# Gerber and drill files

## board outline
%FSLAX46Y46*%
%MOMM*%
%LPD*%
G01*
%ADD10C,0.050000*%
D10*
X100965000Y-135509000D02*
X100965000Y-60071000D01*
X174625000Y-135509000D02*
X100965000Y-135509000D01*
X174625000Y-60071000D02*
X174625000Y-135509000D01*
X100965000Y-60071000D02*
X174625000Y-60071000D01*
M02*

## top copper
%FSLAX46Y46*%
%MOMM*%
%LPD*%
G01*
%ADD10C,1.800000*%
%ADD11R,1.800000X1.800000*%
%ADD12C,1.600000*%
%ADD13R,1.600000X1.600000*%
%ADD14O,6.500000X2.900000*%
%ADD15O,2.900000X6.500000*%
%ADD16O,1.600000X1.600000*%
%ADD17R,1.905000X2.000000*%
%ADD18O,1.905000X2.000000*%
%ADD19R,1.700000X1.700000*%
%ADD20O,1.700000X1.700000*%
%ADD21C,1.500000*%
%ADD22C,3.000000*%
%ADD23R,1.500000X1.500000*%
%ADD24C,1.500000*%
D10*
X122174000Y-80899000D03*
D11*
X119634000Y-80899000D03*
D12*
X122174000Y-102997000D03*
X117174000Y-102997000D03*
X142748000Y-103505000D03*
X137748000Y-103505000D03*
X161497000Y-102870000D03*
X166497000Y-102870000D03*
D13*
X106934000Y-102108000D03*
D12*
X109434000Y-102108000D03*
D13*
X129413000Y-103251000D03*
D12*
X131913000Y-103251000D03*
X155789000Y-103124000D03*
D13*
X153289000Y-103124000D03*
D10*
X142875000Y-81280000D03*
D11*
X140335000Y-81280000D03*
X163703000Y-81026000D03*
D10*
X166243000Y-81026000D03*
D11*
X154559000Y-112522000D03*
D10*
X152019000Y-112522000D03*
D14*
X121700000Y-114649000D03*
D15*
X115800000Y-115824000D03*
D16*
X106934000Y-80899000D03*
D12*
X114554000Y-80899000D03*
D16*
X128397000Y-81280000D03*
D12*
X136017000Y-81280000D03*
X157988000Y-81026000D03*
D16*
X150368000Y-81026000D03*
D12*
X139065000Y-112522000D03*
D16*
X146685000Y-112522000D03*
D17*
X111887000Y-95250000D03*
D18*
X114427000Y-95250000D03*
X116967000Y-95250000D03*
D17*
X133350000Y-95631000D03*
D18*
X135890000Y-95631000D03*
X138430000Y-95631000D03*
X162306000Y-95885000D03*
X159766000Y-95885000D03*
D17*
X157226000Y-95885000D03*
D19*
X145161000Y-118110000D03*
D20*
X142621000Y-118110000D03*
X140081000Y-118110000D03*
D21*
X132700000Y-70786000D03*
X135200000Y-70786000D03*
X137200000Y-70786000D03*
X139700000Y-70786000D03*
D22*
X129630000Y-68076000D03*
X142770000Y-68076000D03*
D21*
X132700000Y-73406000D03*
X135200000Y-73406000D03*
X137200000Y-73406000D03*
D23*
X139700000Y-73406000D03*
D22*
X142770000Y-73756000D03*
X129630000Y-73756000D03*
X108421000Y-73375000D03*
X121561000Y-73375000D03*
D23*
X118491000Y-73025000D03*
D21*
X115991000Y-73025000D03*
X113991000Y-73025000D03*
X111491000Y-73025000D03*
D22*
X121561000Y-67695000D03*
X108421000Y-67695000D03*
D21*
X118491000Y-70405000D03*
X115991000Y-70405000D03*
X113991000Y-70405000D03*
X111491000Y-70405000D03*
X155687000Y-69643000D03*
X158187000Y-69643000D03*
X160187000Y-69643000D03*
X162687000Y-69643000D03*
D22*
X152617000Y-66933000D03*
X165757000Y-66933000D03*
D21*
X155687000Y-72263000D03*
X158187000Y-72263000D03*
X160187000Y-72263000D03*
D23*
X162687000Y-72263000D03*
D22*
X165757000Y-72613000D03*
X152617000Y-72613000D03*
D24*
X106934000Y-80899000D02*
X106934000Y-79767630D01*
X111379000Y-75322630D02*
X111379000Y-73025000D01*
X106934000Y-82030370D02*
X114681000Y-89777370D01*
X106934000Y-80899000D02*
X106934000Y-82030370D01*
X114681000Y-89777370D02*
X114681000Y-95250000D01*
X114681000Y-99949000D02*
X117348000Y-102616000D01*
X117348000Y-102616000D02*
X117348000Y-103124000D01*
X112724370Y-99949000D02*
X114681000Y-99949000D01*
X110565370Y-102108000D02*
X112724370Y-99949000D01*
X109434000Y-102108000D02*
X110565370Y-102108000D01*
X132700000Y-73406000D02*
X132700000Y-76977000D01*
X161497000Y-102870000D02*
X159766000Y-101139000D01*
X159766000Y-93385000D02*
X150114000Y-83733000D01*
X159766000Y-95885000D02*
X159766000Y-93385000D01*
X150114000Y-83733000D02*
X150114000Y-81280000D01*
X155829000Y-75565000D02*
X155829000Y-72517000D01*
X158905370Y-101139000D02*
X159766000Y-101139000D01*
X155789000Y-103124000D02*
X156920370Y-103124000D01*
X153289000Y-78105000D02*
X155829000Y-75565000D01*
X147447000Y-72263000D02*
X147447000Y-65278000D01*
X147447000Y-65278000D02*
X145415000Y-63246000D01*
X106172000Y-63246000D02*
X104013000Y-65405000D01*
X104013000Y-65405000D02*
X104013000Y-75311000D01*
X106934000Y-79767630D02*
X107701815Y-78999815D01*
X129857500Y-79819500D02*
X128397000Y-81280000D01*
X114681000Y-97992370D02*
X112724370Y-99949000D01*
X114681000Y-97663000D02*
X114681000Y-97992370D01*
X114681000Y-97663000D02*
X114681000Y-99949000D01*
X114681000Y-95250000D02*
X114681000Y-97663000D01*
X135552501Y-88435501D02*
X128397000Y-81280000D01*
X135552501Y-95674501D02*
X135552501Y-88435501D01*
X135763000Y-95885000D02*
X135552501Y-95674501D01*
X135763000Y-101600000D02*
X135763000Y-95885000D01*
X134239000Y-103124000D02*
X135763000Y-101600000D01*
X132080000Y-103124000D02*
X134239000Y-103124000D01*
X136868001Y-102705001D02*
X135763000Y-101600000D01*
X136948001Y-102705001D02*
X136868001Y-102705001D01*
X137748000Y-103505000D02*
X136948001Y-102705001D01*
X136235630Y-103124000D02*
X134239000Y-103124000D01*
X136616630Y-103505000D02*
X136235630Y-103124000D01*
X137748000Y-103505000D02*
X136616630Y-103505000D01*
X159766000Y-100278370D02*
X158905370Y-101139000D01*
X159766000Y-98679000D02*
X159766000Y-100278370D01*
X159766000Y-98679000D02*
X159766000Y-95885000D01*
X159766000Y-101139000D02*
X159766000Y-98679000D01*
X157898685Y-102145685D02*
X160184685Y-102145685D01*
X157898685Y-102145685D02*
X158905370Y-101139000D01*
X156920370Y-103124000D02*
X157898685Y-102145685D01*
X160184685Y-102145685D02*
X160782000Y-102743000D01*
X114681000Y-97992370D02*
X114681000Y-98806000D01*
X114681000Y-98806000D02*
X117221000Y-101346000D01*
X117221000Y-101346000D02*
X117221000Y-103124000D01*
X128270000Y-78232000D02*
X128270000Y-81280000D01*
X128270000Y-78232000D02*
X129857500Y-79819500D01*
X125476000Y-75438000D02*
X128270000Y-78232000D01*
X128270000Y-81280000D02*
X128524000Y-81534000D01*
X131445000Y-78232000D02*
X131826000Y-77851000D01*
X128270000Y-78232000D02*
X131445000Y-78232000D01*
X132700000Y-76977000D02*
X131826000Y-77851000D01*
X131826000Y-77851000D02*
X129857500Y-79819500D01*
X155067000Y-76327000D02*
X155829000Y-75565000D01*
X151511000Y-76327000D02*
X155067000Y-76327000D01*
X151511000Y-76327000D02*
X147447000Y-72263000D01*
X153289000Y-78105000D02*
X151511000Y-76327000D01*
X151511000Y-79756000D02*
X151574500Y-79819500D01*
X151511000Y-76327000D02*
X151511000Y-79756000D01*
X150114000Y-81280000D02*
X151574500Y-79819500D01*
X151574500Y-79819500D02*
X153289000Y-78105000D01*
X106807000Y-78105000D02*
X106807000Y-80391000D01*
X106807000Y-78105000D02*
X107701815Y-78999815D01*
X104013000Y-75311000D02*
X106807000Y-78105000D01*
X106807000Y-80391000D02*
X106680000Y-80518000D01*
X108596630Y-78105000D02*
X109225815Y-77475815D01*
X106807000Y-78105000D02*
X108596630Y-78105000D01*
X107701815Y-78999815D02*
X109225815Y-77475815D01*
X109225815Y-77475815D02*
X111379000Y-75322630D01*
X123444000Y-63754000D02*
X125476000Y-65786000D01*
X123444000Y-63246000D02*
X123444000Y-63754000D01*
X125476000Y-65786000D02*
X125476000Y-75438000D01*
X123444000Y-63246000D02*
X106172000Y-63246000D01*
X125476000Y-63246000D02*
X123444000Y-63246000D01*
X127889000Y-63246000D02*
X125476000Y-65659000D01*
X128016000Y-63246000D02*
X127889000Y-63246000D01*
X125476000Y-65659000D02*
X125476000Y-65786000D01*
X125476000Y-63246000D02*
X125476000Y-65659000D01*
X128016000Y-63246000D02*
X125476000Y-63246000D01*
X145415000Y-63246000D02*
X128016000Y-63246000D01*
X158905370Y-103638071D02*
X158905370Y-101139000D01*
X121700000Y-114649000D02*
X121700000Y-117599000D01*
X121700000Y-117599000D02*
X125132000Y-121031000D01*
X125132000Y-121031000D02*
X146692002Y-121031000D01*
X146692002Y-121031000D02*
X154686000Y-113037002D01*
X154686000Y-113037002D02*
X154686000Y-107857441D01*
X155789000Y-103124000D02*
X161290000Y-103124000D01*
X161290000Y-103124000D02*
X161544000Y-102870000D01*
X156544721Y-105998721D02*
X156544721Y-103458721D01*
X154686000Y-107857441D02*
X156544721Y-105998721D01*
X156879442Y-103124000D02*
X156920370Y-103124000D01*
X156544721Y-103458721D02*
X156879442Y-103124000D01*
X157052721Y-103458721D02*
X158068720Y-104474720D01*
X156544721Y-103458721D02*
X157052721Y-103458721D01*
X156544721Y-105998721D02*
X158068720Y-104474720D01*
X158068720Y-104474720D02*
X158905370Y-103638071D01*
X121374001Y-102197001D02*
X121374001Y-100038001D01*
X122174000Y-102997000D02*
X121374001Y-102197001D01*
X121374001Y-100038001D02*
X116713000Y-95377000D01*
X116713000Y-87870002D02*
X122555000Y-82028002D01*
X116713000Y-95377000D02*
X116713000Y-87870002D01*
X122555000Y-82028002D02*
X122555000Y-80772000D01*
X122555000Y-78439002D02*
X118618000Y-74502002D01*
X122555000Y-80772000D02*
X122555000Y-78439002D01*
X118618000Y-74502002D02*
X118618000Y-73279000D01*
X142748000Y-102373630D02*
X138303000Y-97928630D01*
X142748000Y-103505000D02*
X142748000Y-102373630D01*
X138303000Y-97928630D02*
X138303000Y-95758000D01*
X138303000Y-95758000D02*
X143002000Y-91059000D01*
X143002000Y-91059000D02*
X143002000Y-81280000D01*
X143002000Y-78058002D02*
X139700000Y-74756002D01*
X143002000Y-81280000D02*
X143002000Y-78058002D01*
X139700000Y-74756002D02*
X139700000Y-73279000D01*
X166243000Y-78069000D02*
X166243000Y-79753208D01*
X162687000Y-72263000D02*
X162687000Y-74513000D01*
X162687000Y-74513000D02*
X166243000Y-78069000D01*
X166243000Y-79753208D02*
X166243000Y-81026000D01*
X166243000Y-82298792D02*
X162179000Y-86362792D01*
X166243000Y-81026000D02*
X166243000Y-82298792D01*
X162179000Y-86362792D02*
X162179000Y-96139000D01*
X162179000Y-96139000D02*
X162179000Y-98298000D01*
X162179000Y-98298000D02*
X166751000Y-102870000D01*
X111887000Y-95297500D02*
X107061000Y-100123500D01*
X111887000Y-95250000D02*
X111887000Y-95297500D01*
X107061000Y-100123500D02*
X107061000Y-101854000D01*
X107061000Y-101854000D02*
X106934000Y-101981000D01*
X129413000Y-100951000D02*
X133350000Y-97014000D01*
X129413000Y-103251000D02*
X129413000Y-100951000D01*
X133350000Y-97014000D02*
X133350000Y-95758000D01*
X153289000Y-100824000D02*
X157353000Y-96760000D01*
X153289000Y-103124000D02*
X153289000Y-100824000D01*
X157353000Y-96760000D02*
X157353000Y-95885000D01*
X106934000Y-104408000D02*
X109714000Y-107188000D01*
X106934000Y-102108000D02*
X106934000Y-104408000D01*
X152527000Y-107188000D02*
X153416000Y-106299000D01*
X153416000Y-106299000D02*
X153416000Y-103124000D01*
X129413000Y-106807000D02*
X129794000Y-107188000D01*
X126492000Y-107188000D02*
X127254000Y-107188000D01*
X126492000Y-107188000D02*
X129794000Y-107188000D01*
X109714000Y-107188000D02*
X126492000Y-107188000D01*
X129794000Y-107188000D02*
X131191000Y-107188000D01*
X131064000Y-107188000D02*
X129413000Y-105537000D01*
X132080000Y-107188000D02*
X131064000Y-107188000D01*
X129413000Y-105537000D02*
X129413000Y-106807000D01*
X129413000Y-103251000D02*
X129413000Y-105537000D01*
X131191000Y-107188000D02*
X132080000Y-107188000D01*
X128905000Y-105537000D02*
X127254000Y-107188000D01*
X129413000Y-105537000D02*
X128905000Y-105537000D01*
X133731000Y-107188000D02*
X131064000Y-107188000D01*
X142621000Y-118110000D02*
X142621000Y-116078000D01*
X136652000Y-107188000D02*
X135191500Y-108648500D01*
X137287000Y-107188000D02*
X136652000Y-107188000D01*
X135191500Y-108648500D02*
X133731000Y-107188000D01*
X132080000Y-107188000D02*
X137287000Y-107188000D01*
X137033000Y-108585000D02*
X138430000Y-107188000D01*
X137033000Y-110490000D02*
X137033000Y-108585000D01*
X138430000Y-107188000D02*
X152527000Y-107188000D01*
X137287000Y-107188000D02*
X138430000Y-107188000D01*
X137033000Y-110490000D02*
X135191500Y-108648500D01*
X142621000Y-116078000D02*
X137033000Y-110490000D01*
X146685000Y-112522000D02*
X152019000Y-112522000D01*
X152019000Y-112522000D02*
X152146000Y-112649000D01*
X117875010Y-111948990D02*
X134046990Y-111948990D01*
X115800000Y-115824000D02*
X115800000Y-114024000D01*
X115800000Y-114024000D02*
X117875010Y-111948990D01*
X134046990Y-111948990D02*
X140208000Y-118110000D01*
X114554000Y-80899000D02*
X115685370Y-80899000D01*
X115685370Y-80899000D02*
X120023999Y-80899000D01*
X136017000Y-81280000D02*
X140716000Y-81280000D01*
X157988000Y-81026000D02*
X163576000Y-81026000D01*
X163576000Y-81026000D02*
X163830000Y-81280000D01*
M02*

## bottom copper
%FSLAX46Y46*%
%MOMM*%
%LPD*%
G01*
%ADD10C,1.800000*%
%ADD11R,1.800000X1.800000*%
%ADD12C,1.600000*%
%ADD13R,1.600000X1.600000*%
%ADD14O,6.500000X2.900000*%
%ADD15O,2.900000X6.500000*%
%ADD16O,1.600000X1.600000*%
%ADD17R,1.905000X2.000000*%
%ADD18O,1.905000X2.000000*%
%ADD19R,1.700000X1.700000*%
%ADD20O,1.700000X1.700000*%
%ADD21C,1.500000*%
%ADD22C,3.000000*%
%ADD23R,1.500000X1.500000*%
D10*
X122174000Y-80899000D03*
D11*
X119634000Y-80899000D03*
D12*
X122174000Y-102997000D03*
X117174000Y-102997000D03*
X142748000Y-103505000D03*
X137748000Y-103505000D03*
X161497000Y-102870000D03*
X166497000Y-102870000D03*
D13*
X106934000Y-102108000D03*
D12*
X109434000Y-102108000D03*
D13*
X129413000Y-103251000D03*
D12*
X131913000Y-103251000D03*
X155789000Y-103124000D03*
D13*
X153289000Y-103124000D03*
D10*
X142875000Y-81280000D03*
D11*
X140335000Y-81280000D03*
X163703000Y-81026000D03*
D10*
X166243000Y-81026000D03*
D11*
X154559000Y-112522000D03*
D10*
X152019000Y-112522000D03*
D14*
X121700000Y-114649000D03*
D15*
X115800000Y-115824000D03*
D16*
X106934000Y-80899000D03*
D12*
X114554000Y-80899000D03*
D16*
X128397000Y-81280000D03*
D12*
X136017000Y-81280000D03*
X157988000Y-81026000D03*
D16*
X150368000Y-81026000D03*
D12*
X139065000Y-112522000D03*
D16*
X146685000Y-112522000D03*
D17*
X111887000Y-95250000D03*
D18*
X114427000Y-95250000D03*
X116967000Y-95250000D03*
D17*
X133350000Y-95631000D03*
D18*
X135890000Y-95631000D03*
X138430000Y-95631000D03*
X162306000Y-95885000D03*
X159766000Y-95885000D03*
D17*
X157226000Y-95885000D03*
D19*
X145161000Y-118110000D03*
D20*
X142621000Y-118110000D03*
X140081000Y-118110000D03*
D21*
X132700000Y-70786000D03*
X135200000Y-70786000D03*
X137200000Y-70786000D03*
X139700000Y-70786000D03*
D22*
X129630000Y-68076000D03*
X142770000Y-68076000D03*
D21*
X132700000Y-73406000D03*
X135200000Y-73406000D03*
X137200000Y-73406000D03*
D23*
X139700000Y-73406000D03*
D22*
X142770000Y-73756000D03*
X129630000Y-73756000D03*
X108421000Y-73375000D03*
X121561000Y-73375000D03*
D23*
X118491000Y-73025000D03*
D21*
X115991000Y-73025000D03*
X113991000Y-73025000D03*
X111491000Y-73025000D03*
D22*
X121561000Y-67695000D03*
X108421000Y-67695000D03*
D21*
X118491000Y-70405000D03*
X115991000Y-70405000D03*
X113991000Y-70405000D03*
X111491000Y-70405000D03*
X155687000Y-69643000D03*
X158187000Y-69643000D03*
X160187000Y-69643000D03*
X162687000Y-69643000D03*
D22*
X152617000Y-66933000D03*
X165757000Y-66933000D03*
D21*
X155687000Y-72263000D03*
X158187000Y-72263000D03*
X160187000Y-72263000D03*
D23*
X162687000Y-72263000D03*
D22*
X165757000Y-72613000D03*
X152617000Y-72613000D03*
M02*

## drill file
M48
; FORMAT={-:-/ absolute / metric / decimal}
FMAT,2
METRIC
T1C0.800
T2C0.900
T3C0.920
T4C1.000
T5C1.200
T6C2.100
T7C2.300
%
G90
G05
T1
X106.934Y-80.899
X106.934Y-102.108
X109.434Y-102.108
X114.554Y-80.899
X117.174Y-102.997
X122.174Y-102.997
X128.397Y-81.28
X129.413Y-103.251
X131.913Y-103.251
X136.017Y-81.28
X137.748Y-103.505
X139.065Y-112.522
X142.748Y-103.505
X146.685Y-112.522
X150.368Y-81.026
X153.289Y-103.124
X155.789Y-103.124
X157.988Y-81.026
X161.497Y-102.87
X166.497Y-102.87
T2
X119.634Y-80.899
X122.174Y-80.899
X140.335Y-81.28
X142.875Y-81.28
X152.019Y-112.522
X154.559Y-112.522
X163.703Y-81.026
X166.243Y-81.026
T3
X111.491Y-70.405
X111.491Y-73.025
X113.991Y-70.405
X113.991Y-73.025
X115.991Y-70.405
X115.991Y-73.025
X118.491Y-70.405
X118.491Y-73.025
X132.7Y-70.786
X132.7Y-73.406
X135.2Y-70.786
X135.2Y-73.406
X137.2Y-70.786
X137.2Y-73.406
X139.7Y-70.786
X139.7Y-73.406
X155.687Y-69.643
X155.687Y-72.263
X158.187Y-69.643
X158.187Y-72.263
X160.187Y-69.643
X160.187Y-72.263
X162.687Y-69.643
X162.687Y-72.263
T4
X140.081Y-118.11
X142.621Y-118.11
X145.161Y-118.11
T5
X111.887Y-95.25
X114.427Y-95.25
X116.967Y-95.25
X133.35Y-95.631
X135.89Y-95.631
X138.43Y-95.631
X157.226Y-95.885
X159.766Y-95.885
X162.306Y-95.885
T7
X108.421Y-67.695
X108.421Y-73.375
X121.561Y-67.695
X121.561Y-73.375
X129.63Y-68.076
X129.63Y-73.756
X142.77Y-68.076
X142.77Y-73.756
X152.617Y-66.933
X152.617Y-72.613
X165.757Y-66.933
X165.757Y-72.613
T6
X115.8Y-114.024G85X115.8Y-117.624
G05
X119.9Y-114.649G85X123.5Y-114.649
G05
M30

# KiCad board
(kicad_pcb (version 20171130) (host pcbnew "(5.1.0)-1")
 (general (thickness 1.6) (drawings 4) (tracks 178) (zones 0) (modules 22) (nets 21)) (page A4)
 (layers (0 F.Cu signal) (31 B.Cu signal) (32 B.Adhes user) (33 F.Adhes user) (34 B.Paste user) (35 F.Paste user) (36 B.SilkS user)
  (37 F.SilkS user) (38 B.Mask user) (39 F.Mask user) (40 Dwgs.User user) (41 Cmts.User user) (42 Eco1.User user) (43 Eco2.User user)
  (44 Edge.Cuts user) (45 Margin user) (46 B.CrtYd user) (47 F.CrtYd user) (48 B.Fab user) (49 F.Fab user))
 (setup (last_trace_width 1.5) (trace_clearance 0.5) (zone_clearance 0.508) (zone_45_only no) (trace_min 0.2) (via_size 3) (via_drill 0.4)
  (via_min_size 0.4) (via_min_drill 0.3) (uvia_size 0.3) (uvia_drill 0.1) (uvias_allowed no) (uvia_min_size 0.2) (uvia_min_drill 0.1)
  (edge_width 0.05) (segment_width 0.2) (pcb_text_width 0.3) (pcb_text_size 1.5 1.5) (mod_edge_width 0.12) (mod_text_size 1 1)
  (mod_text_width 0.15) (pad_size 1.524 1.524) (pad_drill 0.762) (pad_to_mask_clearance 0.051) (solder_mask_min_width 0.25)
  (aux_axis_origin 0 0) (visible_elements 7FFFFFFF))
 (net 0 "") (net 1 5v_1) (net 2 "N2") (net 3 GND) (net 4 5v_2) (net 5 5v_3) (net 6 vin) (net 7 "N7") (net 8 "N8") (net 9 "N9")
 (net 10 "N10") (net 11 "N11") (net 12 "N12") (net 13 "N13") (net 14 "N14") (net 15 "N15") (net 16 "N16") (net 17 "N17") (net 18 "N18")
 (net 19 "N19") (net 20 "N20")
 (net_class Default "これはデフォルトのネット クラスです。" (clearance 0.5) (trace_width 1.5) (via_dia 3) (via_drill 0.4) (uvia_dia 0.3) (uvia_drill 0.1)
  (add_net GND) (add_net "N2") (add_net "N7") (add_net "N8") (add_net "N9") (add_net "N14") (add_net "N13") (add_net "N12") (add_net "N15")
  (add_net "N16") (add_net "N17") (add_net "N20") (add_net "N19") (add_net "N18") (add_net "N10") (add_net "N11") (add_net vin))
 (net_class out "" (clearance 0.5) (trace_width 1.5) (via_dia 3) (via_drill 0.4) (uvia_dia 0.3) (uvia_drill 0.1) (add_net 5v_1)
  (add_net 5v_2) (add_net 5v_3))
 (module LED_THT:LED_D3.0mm (layer F.Cu) (at 119.634 80.899)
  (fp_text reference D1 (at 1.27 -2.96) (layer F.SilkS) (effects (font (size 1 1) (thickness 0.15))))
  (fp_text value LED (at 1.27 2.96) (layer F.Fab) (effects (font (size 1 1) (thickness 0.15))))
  (pad 2 thru_hole circle (at 2.54 0) (size 1.8 1.8) (drill 0.9) (layers *.Cu *.Mask) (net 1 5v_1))
  (pad 1 thru_hole rect (at 0 0) (size 1.8 1.8) (drill 0.9) (layers *.Cu *.Mask) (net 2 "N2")))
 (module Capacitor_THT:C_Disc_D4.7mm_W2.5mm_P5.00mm (layer F.Cu) (at 122.174 102.997 180)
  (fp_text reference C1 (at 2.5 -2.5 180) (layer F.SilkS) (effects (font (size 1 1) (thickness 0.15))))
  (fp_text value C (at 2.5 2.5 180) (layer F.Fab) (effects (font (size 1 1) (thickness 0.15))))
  (pad 1 thru_hole circle (at 0 0 180) (size 1.6 1.6) (drill 0.8) (layers *.Cu *.Mask) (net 1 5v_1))
  (pad 2 thru_hole circle (at 5 0 180) (size 1.6 1.6) (drill 0.8) (layers *.Cu *.Mask) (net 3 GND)))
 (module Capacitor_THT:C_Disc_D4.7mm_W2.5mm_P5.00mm (layer F.Cu) (at 142.748 103.505 180)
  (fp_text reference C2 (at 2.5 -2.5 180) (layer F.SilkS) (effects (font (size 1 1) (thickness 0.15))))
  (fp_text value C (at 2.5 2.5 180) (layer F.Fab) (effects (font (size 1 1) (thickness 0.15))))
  (pad 1 thru_hole circle (at 0 0 180) (size 1.6 1.6) (drill 0.8) (layers *.Cu *.Mask) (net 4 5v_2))
  (pad 2 thru_hole circle (at 5 0 180) (size 1.6 1.6) (drill 0.8) (layers *.Cu *.Mask) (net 3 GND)))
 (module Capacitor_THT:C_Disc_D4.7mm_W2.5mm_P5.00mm (layer F.Cu) (at 166.497 102.87 180)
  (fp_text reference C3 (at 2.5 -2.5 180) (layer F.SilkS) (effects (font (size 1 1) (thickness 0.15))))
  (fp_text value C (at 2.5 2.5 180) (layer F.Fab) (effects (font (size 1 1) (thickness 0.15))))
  (pad 2 thru_hole circle (at 5 0 180) (size 1.6 1.6) (drill 0.8) (layers *.Cu *.Mask) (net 3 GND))
  (pad 1 thru_hole circle (at 0 0 180) (size 1.6 1.6) (drill 0.8) (layers *.Cu *.Mask) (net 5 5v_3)))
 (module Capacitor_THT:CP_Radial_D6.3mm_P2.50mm (layer F.Cu) (at 106.934 102.108)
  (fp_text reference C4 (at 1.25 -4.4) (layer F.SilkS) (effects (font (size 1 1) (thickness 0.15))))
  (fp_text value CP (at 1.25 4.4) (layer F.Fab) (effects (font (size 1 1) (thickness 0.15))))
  (pad 1 thru_hole rect (at 0 0) (size 1.6 1.6) (drill 0.8) (layers *.Cu *.Mask) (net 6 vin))
  (pad 2 thru_hole circle (at 2.5 0) (size 1.6 1.6) (drill 0.8) (layers *.Cu *.Mask) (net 3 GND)))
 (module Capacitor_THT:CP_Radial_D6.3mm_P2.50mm (layer F.Cu) (at 129.413 103.251)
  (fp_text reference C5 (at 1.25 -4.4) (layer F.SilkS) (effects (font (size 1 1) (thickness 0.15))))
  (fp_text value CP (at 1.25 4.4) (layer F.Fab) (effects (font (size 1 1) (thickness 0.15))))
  (pad 1 thru_hole rect (at 0 0) (size 1.6 1.6) (drill 0.8) (layers *.Cu *.Mask) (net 6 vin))
  (pad 2 thru_hole circle (at 2.5 0) (size 1.6 1.6) (drill 0.8) (layers *.Cu *.Mask) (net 3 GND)))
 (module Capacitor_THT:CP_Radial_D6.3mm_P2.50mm (layer F.Cu) (at 153.289 103.124)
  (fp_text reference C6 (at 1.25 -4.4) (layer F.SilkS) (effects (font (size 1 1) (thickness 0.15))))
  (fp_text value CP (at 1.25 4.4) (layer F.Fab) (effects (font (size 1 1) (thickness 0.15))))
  (pad 2 thru_hole circle (at 2.5 0) (size 1.6 1.6) (drill 0.8) (layers *.Cu *.Mask) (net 3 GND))
  (pad 1 thru_hole rect (at 0 0) (size 1.6 1.6) (drill 0.8) (layers *.Cu *.Mask) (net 6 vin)))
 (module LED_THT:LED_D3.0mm (layer F.Cu) (at 140.335 81.28)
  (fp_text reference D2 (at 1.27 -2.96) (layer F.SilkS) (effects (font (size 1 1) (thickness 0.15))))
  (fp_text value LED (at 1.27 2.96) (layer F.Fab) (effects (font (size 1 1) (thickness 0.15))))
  (pad 2 thru_hole circle (at 2.54 0) (size 1.8 1.8) (drill 0.9) (layers *.Cu *.Mask) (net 4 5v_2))
  (pad 1 thru_hole rect (at 0 0) (size 1.8 1.8) (drill 0.9) (layers *.Cu *.Mask) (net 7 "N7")))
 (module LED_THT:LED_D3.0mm (layer F.Cu) (at 163.703 81.026)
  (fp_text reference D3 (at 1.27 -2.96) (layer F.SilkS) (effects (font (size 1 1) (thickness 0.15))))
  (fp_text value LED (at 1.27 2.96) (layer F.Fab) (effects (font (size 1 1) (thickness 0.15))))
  (pad 1 thru_hole rect (at 0 0) (size 1.8 1.8) (drill 0.9) (layers *.Cu *.Mask) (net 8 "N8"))
  (pad 2 thru_hole circle (at 2.54 0) (size 1.8 1.8) (drill 0.9) (layers *.Cu *.Mask) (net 5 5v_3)))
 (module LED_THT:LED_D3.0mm (layer F.Cu) (at 154.559 112.522 180)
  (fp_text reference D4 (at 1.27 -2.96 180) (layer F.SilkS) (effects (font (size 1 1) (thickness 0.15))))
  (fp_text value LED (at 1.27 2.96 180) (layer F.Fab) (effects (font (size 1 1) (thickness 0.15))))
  (pad 1 thru_hole rect (at 0 0 180) (size 1.8 1.8) (drill 0.9) (layers *.Cu *.Mask) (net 3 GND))
  (pad 2 thru_hole circle (at 2.54 0 180) (size 1.8 1.8) (drill 0.9) (layers *.Cu *.Mask) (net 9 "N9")))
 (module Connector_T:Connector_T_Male (layer F.Cu) (at 114.3 115.824)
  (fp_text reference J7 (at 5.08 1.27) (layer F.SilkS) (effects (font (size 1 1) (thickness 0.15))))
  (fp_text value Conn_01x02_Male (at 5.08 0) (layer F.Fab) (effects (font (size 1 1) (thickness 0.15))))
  (pad 2 thru_hole oval (at 7.4 -1.175) (size 6.5 2.9) (drill oval 5.7 2.1) (layers *.Cu *.Mask) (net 3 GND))
  (pad 1 thru_hole oval (at 1.5 0) (size 2.9 6.5) (drill oval 2.1 5.7) (layers *.Cu *.Mask) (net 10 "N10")))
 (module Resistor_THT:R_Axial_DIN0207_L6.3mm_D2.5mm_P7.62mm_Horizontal (layer F.Cu) (at 114.554 80.899 180)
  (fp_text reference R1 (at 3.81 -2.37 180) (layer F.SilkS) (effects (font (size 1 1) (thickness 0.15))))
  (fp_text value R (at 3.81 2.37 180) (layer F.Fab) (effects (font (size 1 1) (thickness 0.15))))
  (pad 2 thru_hole oval (at 7.62 0 180) (size 1.6 1.6) (drill 0.8) (layers *.Cu *.Mask) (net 3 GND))
  (pad 1 thru_hole circle (at 0 0 180) (size 1.6 1.6) (drill 0.8) (layers *.Cu *.Mask) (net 2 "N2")))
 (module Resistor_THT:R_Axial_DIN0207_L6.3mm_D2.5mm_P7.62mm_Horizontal (layer F.Cu) (at 136.017 81.28 180)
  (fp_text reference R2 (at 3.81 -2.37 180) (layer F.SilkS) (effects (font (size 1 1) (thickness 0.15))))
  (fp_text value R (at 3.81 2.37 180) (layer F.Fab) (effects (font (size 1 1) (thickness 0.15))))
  (pad 2 thru_hole oval (at 7.62 0 180) (size 1.6 1.6) (drill 0.8) (layers *.Cu *.Mask) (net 3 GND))
  (pad 1 thru_hole circle (at 0 0 180) (size 1.6 1.6) (drill 0.8) (layers *.Cu *.Mask) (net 7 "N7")))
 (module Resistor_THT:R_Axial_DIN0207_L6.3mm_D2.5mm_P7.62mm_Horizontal (layer F.Cu) (at 157.988 81.026 180)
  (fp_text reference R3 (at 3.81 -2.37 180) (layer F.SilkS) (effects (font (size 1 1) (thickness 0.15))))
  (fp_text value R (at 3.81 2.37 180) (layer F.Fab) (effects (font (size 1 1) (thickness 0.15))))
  (pad 1 thru_hole circle (at 0 0 180) (size 1.6 1.6) (drill 0.8) (layers *.Cu *.Mask) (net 8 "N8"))
  (pad 2 thru_hole oval (at 7.62 0 180) (size 1.6 1.6) (drill 0.8) (layers *.Cu *.Mask) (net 3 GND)))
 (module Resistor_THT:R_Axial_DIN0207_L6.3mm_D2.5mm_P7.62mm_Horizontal (layer F.Cu) (at 139.065 112.522)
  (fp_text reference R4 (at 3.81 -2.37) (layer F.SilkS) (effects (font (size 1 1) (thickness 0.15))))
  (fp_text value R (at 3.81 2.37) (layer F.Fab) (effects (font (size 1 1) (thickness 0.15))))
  (pad 1 thru_hole circle (at 0 0) (size 1.6 1.6) (drill 0.8) (layers *.Cu *.Mask) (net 6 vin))
  (pad 2 thru_hole oval (at 7.62 0) (size 1.6 1.6) (drill 0.8) (layers *.Cu *.Mask) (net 9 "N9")))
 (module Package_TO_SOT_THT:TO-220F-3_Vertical (layer F.Cu) (at 111.887 95.25)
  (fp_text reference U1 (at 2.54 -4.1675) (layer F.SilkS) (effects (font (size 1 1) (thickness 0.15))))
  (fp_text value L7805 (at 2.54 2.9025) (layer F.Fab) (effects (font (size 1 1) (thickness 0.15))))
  (pad 1 thru_hole rect (at 0 0) (size 1.905 2) (drill 1.2) (layers *.Cu *.Mask) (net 6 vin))
  (pad 2 thru_hole oval (at 2.54 0) (size 1.905 2) (drill 1.2) (layers *.Cu *.Mask) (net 3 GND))
  (pad 3 thru_hole oval (at 5.08 0) (size 1.905 2) (drill 1.2) (layers *.Cu *.Mask) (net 1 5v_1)))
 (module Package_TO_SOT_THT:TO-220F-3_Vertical (layer F.Cu) (at 133.35 95.631)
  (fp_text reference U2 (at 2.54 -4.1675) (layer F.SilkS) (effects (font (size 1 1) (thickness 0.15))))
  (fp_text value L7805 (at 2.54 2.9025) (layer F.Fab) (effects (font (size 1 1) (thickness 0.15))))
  (pad 1 thru_hole rect (at 0 0) (size 1.905 2) (drill 1.2) (layers *.Cu *.Mask) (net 6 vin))
  (pad 2 thru_hole oval (at 2.54 0) (size 1.905 2) (drill 1.2) (layers *.Cu *.Mask) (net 3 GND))
  (pad 3 thru_hole oval (at 5.08 0) (size 1.905 2) (drill 1.2) (layers *.Cu *.Mask) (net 4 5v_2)))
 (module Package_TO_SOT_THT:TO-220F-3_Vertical (layer F.Cu) (at 157.226 95.885)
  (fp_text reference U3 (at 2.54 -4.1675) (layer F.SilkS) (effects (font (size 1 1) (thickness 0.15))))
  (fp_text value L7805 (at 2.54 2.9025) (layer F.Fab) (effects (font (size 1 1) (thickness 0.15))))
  (pad 3 thru_hole oval (at 5.08 0) (size 1.905 2) (drill 1.2) (layers *.Cu *.Mask) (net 5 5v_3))
  (pad 2 thru_hole oval (at 2.54 0) (size 1.905 2) (drill 1.2) (layers *.Cu *.Mask) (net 3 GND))
  (pad 1 thru_hole rect (at 0 0) (size 1.905 2) (drill 1.2) (layers *.Cu *.Mask) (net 6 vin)))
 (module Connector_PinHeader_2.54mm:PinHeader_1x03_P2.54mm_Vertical (layer F.Cu) (at 145.161 118.11 270)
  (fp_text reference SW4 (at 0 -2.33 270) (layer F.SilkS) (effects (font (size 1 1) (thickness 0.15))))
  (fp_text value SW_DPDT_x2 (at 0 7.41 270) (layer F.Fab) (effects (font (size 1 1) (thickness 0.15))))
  (pad 1 thru_hole rect (at 0 0 270) (size 1.7 1.7) (drill 1) (layers *.Cu *.Mask) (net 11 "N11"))
  (pad 2 thru_hole oval (at 0 2.54 270) (size 1.7 1.7) (drill 1) (layers *.Cu *.Mask) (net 6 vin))
  (pad 3 thru_hole oval (at 0 5.08 270) (size 1.7 1.7) (drill 1) (layers *.Cu *.Mask) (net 10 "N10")))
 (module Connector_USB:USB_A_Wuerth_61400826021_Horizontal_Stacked (layer F.Cu) (at 139.7 73.406 180)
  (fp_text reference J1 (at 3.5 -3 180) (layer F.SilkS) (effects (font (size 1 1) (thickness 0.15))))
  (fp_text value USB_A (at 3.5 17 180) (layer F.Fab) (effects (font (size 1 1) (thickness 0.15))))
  (pad 8 thru_hole circle (at 7 2.62 180) (size 1.5 1.5) (drill 0.92) (layers *.Cu *.Mask))
  (pad 7 thru_hole circle (at 4.5 2.62 180) (size 1.5 1.5) (drill 0.92) (layers *.Cu *.Mask))
  (pad 6 thru_hole circle (at 2.5 2.62 180) (size 1.5 1.5) (drill 0.92) (layers *.Cu *.Mask))
  (pad 5 thru_hole circle (at 0 2.62 180) (size 1.5 1.5) (drill 0.92) (layers *.Cu *.Mask) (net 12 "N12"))
  (pad 9 thru_hole circle (at 10.07 5.33 180) (size 3 3) (drill 2.3) (layers *.Cu *.Mask))
  (pad 9 thru_hole circle (at -3.07 5.33 180) (size 3 3) (drill 2.3) (layers *.Cu *.Mask))
  (pad 4 thru_hole circle (at 7 0 180) (size 1.5 1.5) (drill 0.92) (layers *.Cu *.Mask) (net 3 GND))
  (pad 3 thru_hole circle (at 4.5 0 180) (size 1.5 1.5) (drill 0.92) (layers *.Cu *.Mask) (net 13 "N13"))
  (pad 2 thru_hole circle (at 2.5 0 180) (size 1.5 1.5) (drill 0.92) (layers *.Cu *.Mask) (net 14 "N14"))
  (pad 1 thru_hole rect (at 0 0 180) (size 1.5 1.5) (drill 0.92) (layers *.Cu *.Mask) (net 4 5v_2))
  (pad 9 thru_hole circle (at -3.07 -0.35 180) (size 3 3) (drill 2.3) (layers *.Cu *.Mask))
  (pad 9 thru_hole circle (at 10.07 -0.35 180) (size 3 3) (drill 2.3) (layers *.Cu *.Mask)))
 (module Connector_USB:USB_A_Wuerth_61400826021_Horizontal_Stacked (layer F.Cu) (at 118.491 73.025 180)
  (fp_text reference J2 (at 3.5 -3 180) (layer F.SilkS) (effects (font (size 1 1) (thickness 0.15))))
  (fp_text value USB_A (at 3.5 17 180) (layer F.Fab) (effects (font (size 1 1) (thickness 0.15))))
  (pad 9 thru_hole circle (at 10.07 -0.35 180) (size 3 3) (drill 2.3) (layers *.Cu *.Mask))
  (pad 9 thru_hole circle (at -3.07 -0.35 180) (size 3 3) (drill 2.3) (layers *.Cu *.Mask))
  (pad 1 thru_hole rect (at 0 0 180) (size 1.5 1.5) (drill 0.92) (layers *.Cu *.Mask) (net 1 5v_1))
  (pad 2 thru_hole circle (at 2.5 0 180) (size 1.5 1.5) (drill 0.92) (layers *.Cu *.Mask) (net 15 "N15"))
  (pad 3 thru_hole circle (at 4.5 0 180) (size 1.5 1.5) (drill 0.92) (layers *.Cu *.Mask) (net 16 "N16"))
  (pad 4 thru_hole circle (at 7 0 180) (size 1.5 1.5) (drill 0.92) (layers *.Cu *.Mask) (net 3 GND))
  (pad 9 thru_hole circle (at -3.07 5.33 180) (size 3 3) (drill 2.3) (layers *.Cu *.Mask))
  (pad 9 thru_hole circle (at 10.07 5.33 180) (size 3 3) (drill 2.3) (layers *.Cu *.Mask))
  (pad 5 thru_hole circle (at 0 2.62 180) (size 1.5 1.5) (drill 0.92) (layers *.Cu *.Mask) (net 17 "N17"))
  (pad 6 thru_hole circle (at 2.5 2.62 180) (size 1.5 1.5) (drill 0.92) (layers *.Cu *.Mask))
  (pad 7 thru_hole circle (at 4.5 2.62 180) (size 1.5 1.5) (drill 0.92) (layers *.Cu *.Mask))
  (pad 8 thru_hole circle (at 7 2.62 180) (size 1.5 1.5) (drill 0.92) (layers *.Cu *.Mask)))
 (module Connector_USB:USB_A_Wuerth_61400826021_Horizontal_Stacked (layer F.Cu) (at 162.687 72.263 180)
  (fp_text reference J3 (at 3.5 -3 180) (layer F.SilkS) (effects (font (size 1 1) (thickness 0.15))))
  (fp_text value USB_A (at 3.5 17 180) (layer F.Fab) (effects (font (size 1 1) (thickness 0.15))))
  (pad 8 thru_hole circle (at 7 2.62 180) (size 1.5 1.5) (drill 0.92) (layers *.Cu *.Mask))
  (pad 7 thru_hole circle (at 4.5 2.62 180) (size 1.5 1.5) (drill 0.92) (layers *.Cu *.Mask))
  (pad 6 thru_hole circle (at 2.5 2.62 180) (size 1.5 1.5) (drill 0.92) (layers *.Cu *.Mask))
  (pad 5 thru_hole circle (at 0 2.62 180) (size 1.5 1.5) (drill 0.92) (layers *.Cu *.Mask) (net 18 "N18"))
  (pad 9 thru_hole circle (at 10.07 5.33 180) (size 3 3) (drill 2.3) (layers *.Cu *.Mask))
  (pad 9 thru_hole circle (at -3.07 5.33 180) (size 3 3) (drill 2.3) (layers *.Cu *.Mask))
  (pad 4 thru_hole circle (at 7 0 180) (size 1.5 1.5) (drill 0.92) (layers *.Cu *.Mask) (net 3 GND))
  (pad 3 thru_hole circle (at 4.5 0 180) (size 1.5 1.5) (drill 0.92) (layers *.Cu *.Mask) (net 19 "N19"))
  (pad 2 thru_hole circle (at 2.5 0 180) (size 1.5 1.5) (drill 0.92) (layers *.Cu *.Mask) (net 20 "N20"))
  (pad 1 thru_hole rect (at 0 0 180) (size 1.5 1.5) (drill 0.92) (layers *.Cu *.Mask) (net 5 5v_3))
  (pad 9 thru_hole circle (at -3.07 -0.35 180) (size 3 3) (drill 2.3) (layers *.Cu *.Mask))
  (pad 9 thru_hole circle (at 10.07 -0.35 180) (size 3 3) (drill 2.3) (layers *.Cu *.Mask)))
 (gr_line (start 100.965 135.509) (end 100.965 60.071) (layer Edge.Cuts) (width 0.05))
 (gr_line (start 174.625 135.509) (end 100.965 135.509) (layer Edge.Cuts) (width 0.05))
 (gr_line (start 174.625 60.071) (end 174.625 135.509) (layer Edge.Cuts) (width 0.05))
 (gr_line (start 100.965 60.071) (end 174.625 60.071) (layer Edge.Cuts) (width 0.05))
 (segment (start 106.934 80.899) (end 106.934 79.76763) (width 1.5) (layer F.Cu) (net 3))
 (segment (start 111.379 75.32263) (end 111.379 73.025) (width 1.5) (layer F.Cu) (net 3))
 (segment (start 106.934 82.03037) (end 114.681 89.77737) (width 1.5) (layer F.Cu) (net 3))
 (segment (start 106.934 80.899) (end 106.934 82.03037) (width 1.5) (layer F.Cu) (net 3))
 (segment (start 114.681 89.77737) (end 114.681 95.25) (width 1.5) (layer F.Cu) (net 3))
 (segment (start 114.681 99.949) (end 117.348 102.616) (width 1.5) (layer F.Cu) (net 3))
 (segment (start 117.348 102.616) (end 117.348 103.124) (width 1.5) (layer F.Cu) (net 3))
 (segment (start 112.72437 99.949) (end 114.681 99.949) (width 1.5) (layer F.Cu) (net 3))
 (segment (start 110.56537 102.108) (end 112.72437 99.949) (width 1.5) (layer F.Cu) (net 3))
 (segment (start 109.434 102.108) (end 110.56537 102.108) (width 1.5) (layer F.Cu) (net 3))
 (segment (start 132.7 73.406) (end 132.7 76.977) (width 1.5) (layer F.Cu) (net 3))
 (segment (start 161.497 102.87) (end 159.766 101.139) (width 1.5) (layer F.Cu) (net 3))
 (segment (start 159.766 93.385) (end 150.114 83.733) (width 1.5) (layer F.Cu) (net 3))
 (segment (start 159.766 95.885) (end 159.766 93.385) (width 1.5) (layer F.Cu) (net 3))
 (segment (start 150.114 83.733) (end 150.114 81.28) (width 1.5) (layer F.Cu) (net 3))
 (segment (start 155.829 75.565) (end 155.829 72.517) (width 1.5) (layer F.Cu) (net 3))
 (segment (start 158.90537 101.139) (end 159.766 101.139) (width 1.5) (layer F.Cu) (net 3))
 (segment (start 155.789 103.124) (end 156.92037 103.124) (width 1.5) (layer F.Cu) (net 3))
 (segment (start 153.289 78.105) (end 155.829 75.565) (width 1.5) (layer F.Cu) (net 3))
 (segment (start 147.447 72.263) (end 147.447 65.278) (width 1.5) (layer F.Cu) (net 3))
 (segment (start 147.447 65.278) (end 145.415 63.246) (width 1.5) (layer F.Cu) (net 3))
 (segment (start 106.172 63.246) (end 104.013 65.405) (width 1.5) (layer F.Cu) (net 3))
 (segment (start 104.013 65.405) (end 104.013 75.311) (width 1.5) (layer F.Cu) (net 3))
 (segment (start 106.934 79.76763) (end 107.701815 78.999815) (width 1.5) (layer F.Cu) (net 3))
 (segment (start 129.8575 79.8195) (end 128.397 81.28) (width 1.5) (layer F.Cu) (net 3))
 (segment (start 114.681 97.99237) (end 112.72437 99.949) (width 1.5) (layer F.Cu) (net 3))
 (segment (start 114.681 97.663) (end 114.681 97.99237) (width 1.5) (layer F.Cu) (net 3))
 (segment (start 114.681 97.663) (end 114.681 99.949) (width 1.5) (layer F.Cu) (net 3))
 (segment (start 114.681 95.25) (end 114.681 97.663) (width 1.5) (layer F.Cu) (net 3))
 (segment (start 135.552501 88.435501) (end 128.397 81.28) (width 1.5) (layer F.Cu) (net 3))
 (segment (start 135.552501 95.674501) (end 135.552501 88.435501) (width 1.5) (layer F.Cu) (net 3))
 (segment (start 135.763 95.885) (end 135.552501 95.674501) (width 1.5) (layer F.Cu) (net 3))
 (segment (start 135.763 101.6) (end 135.763 95.885) (width 1.5) (layer F.Cu) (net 3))
 (segment (start 134.239 103.124) (end 135.763 101.6) (width 1.5) (layer F.Cu) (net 3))
 (segment (start 132.08 103.124) (end 134.239 103.124) (width 1.5) (layer F.Cu) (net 3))
 (segment (start 136.868001 102.705001) (end 135.763 101.6) (width 1.5) (layer F.Cu) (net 3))
 (segment (start 136.948001 102.705001) (end 136.868001 102.705001) (width 1.5) (layer F.Cu) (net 3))
 (segment (start 137.748 103.505) (end 136.948001 102.705001) (width 1.5) (layer F.Cu) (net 3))
 (segment (start 136.23563 103.124) (end 134.239 103.124) (width 1.5) (layer F.Cu) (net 3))
 (segment (start 136.61663 103.505) (end 136.23563 103.124) (width 1.5) (layer F.Cu) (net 3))
 (segment (start 137.748 103.505) (end 136.61663 103.505) (width 1.5) (layer F.Cu) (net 3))
 (segment (start 159.766 100.27837) (end 158.90537 101.139) (width 1.5) (layer F.Cu) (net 3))
 (segment (start 159.766 98.679) (end 159.766 100.27837) (width 1.5) (layer F.Cu) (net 3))
 (segment (start 159.766 98.679) (end 159.766 95.885) (width 1.5) (layer F.Cu) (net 3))
 (segment (start 159.766 101.139) (end 159.766 98.679) (width 1.5) (layer F.Cu) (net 3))
 (segment (start 157.898685 102.145685) (end 160.184685 102.145685) (width 1.5) (layer F.Cu) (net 3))
 (segment (start 157.898685 102.145685) (end 158.90537 101.139) (width 1.5) (layer F.Cu) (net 3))
 (segment (start 156.92037 103.124) (end 157.898685 102.145685) (width 1.5) (layer F.Cu) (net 3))
 (segment (start 160.184685 102.145685) (end 160.782 102.743) (width 1.5) (layer F.Cu) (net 3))
 (segment (start 114.681 97.99237) (end 114.681 98.806) (width 1.5) (layer F.Cu) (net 3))
 (segment (start 114.681 98.806) (end 117.221 101.346) (width 1.5) (layer F.Cu) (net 3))
 (segment (start 117.221 101.346) (end 117.221 103.124) (width 1.5) (layer F.Cu) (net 3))
 (segment (start 128.27 78.232) (end 128.27 81.28) (width 1.5) (layer F.Cu) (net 3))
 (segment (start 128.27 78.232) (end 129.8575 79.8195) (width 1.5) (layer F.Cu) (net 3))
 (segment (start 125.476 75.438) (end 128.27 78.232) (width 1.5) (layer F.Cu) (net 3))
 (segment (start 128.27 81.28) (end 128.524 81.534) (width 1.5) (layer F.Cu) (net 3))
 (segment (start 131.445 78.232) (end 131.826 77.851) (width 1.5) (layer F.Cu) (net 3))
 (segment (start 128.27 78.232) (end 131.445 78.232) (width 1.5) (layer F.Cu) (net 3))
 (segment (start 132.7 76.977) (end 131.826 77.851) (width 1.5) (layer F.Cu) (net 3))
 (segment (start 131.826 77.851) (end 129.8575 79.8195) (width 1.5) (layer F.Cu) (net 3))
 (segment (start 155.067 76.327) (end 155.829 75.565) (width 1.5) (layer F.Cu) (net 3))
 (segment (start 151.511 76.327) (end 155.067 76.327) (width 1.5) (layer F.Cu) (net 3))
 (segment (start 151.511 76.327) (end 147.447 72.263) (width 1.5) (layer F.Cu) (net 3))
 (segment (start 153.289 78.105) (end 151.511 76.327) (width 1.5) (layer F.Cu) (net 3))
 (segment (start 151.511 79.756) (end 151.5745 79.8195) (width 1.5) (layer F.Cu) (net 3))
 (segment (start 151.511 76.327) (end 151.511 79.756) (width 1.5) (layer F.Cu) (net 3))
 (segment (start 150.114 81.28) (end 151.5745 79.8195) (width 1.5) (layer F.Cu) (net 3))
 (segment (start 151.5745 79.8195) (end 153.289 78.105) (width 1.5) (layer F.Cu) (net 3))
 (segment (start 106.807 78.105) (end 106.807 80.391) (width 1.5) (layer F.Cu) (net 3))
 (segment (start 106.807 78.105) (end 107.701815 78.999815) (width 1.5) (layer F.Cu) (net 3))
 (segment (start 104.013 75.311) (end 106.807 78.105) (width 1.5) (layer F.Cu) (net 3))
 (segment (start 106.807 80.391) (end 106.68 80.518) (width 1.5) (layer F.Cu) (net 3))
 (segment (start 108.59663 78.105) (end 109.225815 77.475815) (width 1.5) (layer F.Cu) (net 3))
 (segment (start 106.807 78.105) (end 108.59663 78.105) (width 1.5) (layer F.Cu) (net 3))
 (segment (start 107.701815 78.999815) (end 109.225815 77.475815) (width 1.5) (layer F.Cu) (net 3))
 (segment (start 109.225815 77.475815) (end 111.379 75.32263) (width 1.5) (layer F.Cu) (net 3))
 (segment (start 123.444 63.754) (end 125.476 65.786) (width 1.5) (layer F.Cu) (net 3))
 (segment (start 123.444 63.246) (end 123.444 63.754) (width 1.5) (layer F.Cu) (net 3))
 (segment (start 125.476 65.786) (end 125.476 75.438) (width 1.5) (layer F.Cu) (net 3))
 (segment (start 123.444 63.246) (end 106.172 63.246) (width 1.5) (layer F.Cu) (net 3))
 (segment (start 125.476 63.246) (end 123.444 63.246) (width 1.5) (layer F.Cu) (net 3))
 (segment (start 127.889 63.246) (end 125.476 65.659) (width 1.5) (layer F.Cu) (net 3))
 (segment (start 128.016 63.246) (end 127.889 63.246) (width 1.5) (layer F.Cu) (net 3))
 (segment (start 125.476 65.659) (end 125.476 65.786) (width 1.5) (layer F.Cu) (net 3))
 (segment (start 125.476 63.246) (end 125.476 65.659) (width 1.5) (layer F.Cu) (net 3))
 (segment (start 128.016 63.246) (end 125.476 63.246) (width 1.5) (layer F.Cu) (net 3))
 (segment (start 145.415 63.246) (end 128.016 63.246) (width 1.5) (layer F.Cu) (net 3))
 (segment (start 158.90537 103.638071) (end 158.90537 101.139) (width 1.5) (layer F.Cu) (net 3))
 (segment (start 121.7 114.649) (end 121.7 117.599) (width 1.5) (layer F.Cu) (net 3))
 (segment (start 121.7 117.599) (end 125.132 121.031) (width 1.5) (layer F.Cu) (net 3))
 (segment (start 125.132 121.031) (end 146.692002 121.031) (width 1.5) (layer F.Cu) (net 3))
 (segment (start 146.692002 121.031) (end 154.686 113.037002) (width 1.5) (layer F.Cu) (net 3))
 (segment (start 154.686 113.037002) (end 154.686 107.857441) (width 1.5) (layer F.Cu) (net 3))
 (segment (start 155.789 103.124) (end 161.29 103.124) (width 1.5) (layer F.Cu) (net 3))
 (segment (start 161.29 103.124) (end 161.544 102.87) (width 1.5) (layer F.Cu) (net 3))
 (segment (start 156.544721 105.998721) (end 156.544721 103.458721) (width 1.5) (layer F.Cu) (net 3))
 (segment (start 154.686 107.857441) (end 156.544721 105.998721) (width 1.5) (layer F.Cu) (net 3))
 (segment (start 156.879442 103.124) (end 156.92037 103.124) (width 1.5) (layer F.Cu) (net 3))
 (segment (start 156.544721 103.458721) (end 156.879442 103.124) (width 1.5) (layer F.Cu) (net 3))
 (segment (start 157.052721 103.458721) (end 158.06872 104.47472) (width 1.5) (layer F.Cu) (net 3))
 (segment (start 156.544721 103.458721) (end 157.052721 103.458721) (width 1.5) (layer F.Cu) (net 3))
 (segment (start 156.544721 105.998721) (end 158.06872 104.47472) (width 1.5) (layer F.Cu) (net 3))
 (segment (start 158.06872 104.47472) (end 158.90537 103.638071) (width 1.5) (layer F.Cu) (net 3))
 (segment (start 121.374001 102.197001) (end 121.374001 100.038001) (width 1.5) (layer F.Cu) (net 1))
 (segment (start 122.174 102.997) (end 121.374001 102.197001) (width 1.5) (layer F.Cu) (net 1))
 (segment (start 121.374001 100.038001) (end 116.713 95.377) (width 1.5) (layer F.Cu) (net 1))
 (segment (start 116.713 87.870002) (end 122.555 82.028002) (width 1.5) (layer F.Cu) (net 1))
 (segment (start 116.713 95.377) (end 116.713 87.870002) (width 1.5) (layer F.Cu) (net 1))
 (segment (start 122.555 82.028002) (end 122.555 80.772) (width 1.5) (layer F.Cu) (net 1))
 (segment (start 122.555 78.439002) (end 118.618 74.502002) (width 1.5) (layer F.Cu) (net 1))
 (segment (start 122.555 80.772) (end 122.555 78.439002) (width 1.5) (layer F.Cu) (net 1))
 (segment (start 118.618 74.502002) (end 118.618 73.279) (width 1.5) (layer F.Cu) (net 1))
 (segment (start 142.748 102.37363) (end 138.303 97.92863) (width 1.5) (layer F.Cu) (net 4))
 (segment (start 142.748 103.505) (end 142.748 102.37363) (width 1.5) (layer F.Cu) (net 4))
 (segment (start 138.303 97.92863) (end 138.303 95.758) (width 1.5) (layer F.Cu) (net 4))
 (segment (start 138.303 95.758) (end 143.002 91.059) (width 1.5) (layer F.Cu) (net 4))
 (segment (start 143.002 91.059) (end 143.002 81.28) (width 1.5) (layer F.Cu) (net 4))
 (segment (start 143.002 78.058002) (end 139.7 74.756002) (width 1.5) (layer F.Cu) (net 4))
 (segment (start 143.002 81.28) (end 143.002 78.058002) (width 1.5) (layer F.Cu) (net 4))
 (segment (start 139.7 74.756002) (end 139.7 73.279) (width 1.5) (layer F.Cu) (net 4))
 (segment (start 166.243 78.069) (end 166.243 79.753208) (width 1.5) (layer F.Cu) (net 5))
 (segment (start 162.687 72.263) (end 162.687 74.513) (width 1.5) (layer F.Cu) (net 5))
 (segment (start 162.687 74.513) (end 166.243 78.069) (width 1.5) (layer F.Cu) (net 5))
 (segment (start 166.243 79.753208) (end 166.243 81.026) (width 1.5) (layer F.Cu) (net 5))
 (segment (start 166.243 82.298792) (end 162.179 86.362792) (width 1.5) (layer F.Cu) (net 5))
 (segment (start 166.243 81.026) (end 166.243 82.298792) (width 1.5) (layer F.Cu) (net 5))
 (segment (start 162.179 86.362792) (end 162.179 96.139) (width 1.5) (layer F.Cu) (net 5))
 (segment (start 162.179 96.139) (end 162.179 98.298) (width 1.5) (layer F.Cu) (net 5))
 (segment (start 162.179 98.298) (end 166.751 102.87) (width 1.5) (layer F.Cu) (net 5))
 (segment (start 111.887 95.2975) (end 107.061 100.1235) (width 1.5) (layer F.Cu) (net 6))
 (segment (start 111.887 95.25) (end 111.887 95.2975) (width 1.5) (layer F.Cu) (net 6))
 (segment (start 107.061 100.1235) (end 107.061 101.854) (width 1.5) (layer F.Cu) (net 6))
 (segment (start 107.061 101.854) (end 106.934 101.981) (width 1.5) (layer F.Cu) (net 6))
 (segment (start 129.413 100.951) (end 133.35 97.014) (width 1.5) (layer F.Cu) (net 6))
 (segment (start 129.413 103.251) (end 129.413 100.951) (width 1.5) (layer F.Cu) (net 6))
 (segment (start 133.35 97.014) (end 133.35 95.758) (width 1.5) (layer F.Cu) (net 6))
 (segment (start 153.289 100.824) (end 157.353 96.76) (width 1.5) (layer F.Cu) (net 6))
 (segment (start 153.289 103.124) (end 153.289 100.824) (width 1.5) (layer F.Cu) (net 6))
 (segment (start 157.353 96.76) (end 157.353 95.885) (width 1.5) (layer F.Cu) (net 6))
 (segment (start 106.934 104.408) (end 109.714 107.188) (width 1.5) (layer F.Cu) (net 6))
 (segment (start 106.934 102.108) (end 106.934 104.408) (width 1.5) (layer F.Cu) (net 6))
 (segment (start 152.527 107.188) (end 153.416 106.299) (width 1.5) (layer F.Cu) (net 6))
 (segment (start 153.416 106.299) (end 153.416 103.124) (width 1.5) (layer F.Cu) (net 6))
 (segment (start 129.413 106.807) (end 129.794 107.188) (width 1.5) (layer F.Cu) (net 6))
 (segment (start 126.492 107.188) (end 127.254 107.188) (width 1.5) (layer F.Cu) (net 6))
 (segment (start 126.492 107.188) (end 129.794 107.188) (width 1.5) (layer F.Cu) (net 6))
 (segment (start 109.714 107.188) (end 126.492 107.188) (width 1.5) (layer F.Cu) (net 6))
 (segment (start 129.794 107.188) (end 131.191 107.188) (width 1.5) (layer F.Cu) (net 6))
 (segment (start 131.064 107.188) (end 129.413 105.537) (width 1.5) (layer F.Cu) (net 6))
 (segment (start 132.08 107.188) (end 131.064 107.188) (width 1.5) (layer F.Cu) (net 6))
 (segment (start 129.413 105.537) (end 129.413 106.807) (width 1.5) (layer F.Cu) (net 6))
 (segment (start 129.413 103.251) (end 129.413 105.537) (width 1.5) (layer F.Cu) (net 6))
 (segment (start 131.191 107.188) (end 132.08 107.188) (width 1.5) (layer F.Cu) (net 6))
 (segment (start 128.905 105.537) (end 127.254 107.188) (width 1.5) (layer F.Cu) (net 6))
 (segment (start 129.413 105.537) (end 128.905 105.537) (width 1.5) (layer F.Cu) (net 6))
 (segment (start 133.731 107.188) (end 131.064 107.188) (width 1.5) (layer F.Cu) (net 6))
 (segment (start 142.621 118.11) (end 142.621 116.078) (width 1.5) (layer F.Cu) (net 6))
 (segment (start 136.652 107.188) (end 135.1915 108.6485) (width 1.5) (layer F.Cu) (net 6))
 (segment (start 137.287 107.188) (end 136.652 107.188) (width 1.5) (layer F.Cu) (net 6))
 (segment (start 135.1915 108.6485) (end 133.731 107.188) (width 1.5) (layer F.Cu) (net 6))
 (segment (start 132.08 107.188) (end 137.287 107.188) (width 1.5) (layer F.Cu) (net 6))
 (segment (start 137.033 108.585) (end 138.43 107.188) (width 1.5) (layer F.Cu) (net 6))
 (segment (start 137.033 110.49) (end 137.033 108.585) (width 1.5) (layer F.Cu) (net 6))
 (segment (start 138.43 107.188) (end 152.527 107.188) (width 1.5) (layer F.Cu) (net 6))
 (segment (start 137.287 107.188) (end 138.43 107.188) (width 1.5) (layer F.Cu) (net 6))
 (segment (start 137.033 110.49) (end 135.1915 108.6485) (width 1.5) (layer F.Cu) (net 6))
 (segment (start 142.621 116.078) (end 137.033 110.49) (width 1.5) (layer F.Cu) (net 6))
 (segment (start 146.685 112.522) (end 152.019 112.522) (width 1.5) (layer F.Cu) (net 9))
 (segment (start 152.019 112.522) (end 152.146 112.649) (width 1.5) (layer F.Cu) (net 9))
 (segment (start 117.87501 111.94899) (end 134.04699 111.94899) (width 1.5) (layer F.Cu) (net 10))
 (segment (start 115.8 115.824) (end 115.8 114.024) (width 1.5) (layer F.Cu) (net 10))
 (segment (start 115.8 114.024) (end 117.87501 111.94899) (width 1.5) (layer F.Cu) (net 10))
 (segment (start 134.04699 111.94899) (end 140.208 118.11) (width 1.5) (layer F.Cu) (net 10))
 (segment (start 114.554 80.899) (end 115.68537 80.899) (width 1.5) (layer F.Cu) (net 2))
 (segment (start 115.68537 80.899) (end 120.023999 80.899) (width 1.5) (layer F.Cu) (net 2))
 (segment (start 136.017 81.28) (end 140.716 81.28) (width 1.5) (layer F.Cu) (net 7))
 (segment (start 157.988 81.026) (end 163.576 81.026) (width 1.5) (layer F.Cu) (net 8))
 (segment (start 163.576 81.026) (end 163.83 81.28) (width 1.5) (layer F.Cu) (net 8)))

